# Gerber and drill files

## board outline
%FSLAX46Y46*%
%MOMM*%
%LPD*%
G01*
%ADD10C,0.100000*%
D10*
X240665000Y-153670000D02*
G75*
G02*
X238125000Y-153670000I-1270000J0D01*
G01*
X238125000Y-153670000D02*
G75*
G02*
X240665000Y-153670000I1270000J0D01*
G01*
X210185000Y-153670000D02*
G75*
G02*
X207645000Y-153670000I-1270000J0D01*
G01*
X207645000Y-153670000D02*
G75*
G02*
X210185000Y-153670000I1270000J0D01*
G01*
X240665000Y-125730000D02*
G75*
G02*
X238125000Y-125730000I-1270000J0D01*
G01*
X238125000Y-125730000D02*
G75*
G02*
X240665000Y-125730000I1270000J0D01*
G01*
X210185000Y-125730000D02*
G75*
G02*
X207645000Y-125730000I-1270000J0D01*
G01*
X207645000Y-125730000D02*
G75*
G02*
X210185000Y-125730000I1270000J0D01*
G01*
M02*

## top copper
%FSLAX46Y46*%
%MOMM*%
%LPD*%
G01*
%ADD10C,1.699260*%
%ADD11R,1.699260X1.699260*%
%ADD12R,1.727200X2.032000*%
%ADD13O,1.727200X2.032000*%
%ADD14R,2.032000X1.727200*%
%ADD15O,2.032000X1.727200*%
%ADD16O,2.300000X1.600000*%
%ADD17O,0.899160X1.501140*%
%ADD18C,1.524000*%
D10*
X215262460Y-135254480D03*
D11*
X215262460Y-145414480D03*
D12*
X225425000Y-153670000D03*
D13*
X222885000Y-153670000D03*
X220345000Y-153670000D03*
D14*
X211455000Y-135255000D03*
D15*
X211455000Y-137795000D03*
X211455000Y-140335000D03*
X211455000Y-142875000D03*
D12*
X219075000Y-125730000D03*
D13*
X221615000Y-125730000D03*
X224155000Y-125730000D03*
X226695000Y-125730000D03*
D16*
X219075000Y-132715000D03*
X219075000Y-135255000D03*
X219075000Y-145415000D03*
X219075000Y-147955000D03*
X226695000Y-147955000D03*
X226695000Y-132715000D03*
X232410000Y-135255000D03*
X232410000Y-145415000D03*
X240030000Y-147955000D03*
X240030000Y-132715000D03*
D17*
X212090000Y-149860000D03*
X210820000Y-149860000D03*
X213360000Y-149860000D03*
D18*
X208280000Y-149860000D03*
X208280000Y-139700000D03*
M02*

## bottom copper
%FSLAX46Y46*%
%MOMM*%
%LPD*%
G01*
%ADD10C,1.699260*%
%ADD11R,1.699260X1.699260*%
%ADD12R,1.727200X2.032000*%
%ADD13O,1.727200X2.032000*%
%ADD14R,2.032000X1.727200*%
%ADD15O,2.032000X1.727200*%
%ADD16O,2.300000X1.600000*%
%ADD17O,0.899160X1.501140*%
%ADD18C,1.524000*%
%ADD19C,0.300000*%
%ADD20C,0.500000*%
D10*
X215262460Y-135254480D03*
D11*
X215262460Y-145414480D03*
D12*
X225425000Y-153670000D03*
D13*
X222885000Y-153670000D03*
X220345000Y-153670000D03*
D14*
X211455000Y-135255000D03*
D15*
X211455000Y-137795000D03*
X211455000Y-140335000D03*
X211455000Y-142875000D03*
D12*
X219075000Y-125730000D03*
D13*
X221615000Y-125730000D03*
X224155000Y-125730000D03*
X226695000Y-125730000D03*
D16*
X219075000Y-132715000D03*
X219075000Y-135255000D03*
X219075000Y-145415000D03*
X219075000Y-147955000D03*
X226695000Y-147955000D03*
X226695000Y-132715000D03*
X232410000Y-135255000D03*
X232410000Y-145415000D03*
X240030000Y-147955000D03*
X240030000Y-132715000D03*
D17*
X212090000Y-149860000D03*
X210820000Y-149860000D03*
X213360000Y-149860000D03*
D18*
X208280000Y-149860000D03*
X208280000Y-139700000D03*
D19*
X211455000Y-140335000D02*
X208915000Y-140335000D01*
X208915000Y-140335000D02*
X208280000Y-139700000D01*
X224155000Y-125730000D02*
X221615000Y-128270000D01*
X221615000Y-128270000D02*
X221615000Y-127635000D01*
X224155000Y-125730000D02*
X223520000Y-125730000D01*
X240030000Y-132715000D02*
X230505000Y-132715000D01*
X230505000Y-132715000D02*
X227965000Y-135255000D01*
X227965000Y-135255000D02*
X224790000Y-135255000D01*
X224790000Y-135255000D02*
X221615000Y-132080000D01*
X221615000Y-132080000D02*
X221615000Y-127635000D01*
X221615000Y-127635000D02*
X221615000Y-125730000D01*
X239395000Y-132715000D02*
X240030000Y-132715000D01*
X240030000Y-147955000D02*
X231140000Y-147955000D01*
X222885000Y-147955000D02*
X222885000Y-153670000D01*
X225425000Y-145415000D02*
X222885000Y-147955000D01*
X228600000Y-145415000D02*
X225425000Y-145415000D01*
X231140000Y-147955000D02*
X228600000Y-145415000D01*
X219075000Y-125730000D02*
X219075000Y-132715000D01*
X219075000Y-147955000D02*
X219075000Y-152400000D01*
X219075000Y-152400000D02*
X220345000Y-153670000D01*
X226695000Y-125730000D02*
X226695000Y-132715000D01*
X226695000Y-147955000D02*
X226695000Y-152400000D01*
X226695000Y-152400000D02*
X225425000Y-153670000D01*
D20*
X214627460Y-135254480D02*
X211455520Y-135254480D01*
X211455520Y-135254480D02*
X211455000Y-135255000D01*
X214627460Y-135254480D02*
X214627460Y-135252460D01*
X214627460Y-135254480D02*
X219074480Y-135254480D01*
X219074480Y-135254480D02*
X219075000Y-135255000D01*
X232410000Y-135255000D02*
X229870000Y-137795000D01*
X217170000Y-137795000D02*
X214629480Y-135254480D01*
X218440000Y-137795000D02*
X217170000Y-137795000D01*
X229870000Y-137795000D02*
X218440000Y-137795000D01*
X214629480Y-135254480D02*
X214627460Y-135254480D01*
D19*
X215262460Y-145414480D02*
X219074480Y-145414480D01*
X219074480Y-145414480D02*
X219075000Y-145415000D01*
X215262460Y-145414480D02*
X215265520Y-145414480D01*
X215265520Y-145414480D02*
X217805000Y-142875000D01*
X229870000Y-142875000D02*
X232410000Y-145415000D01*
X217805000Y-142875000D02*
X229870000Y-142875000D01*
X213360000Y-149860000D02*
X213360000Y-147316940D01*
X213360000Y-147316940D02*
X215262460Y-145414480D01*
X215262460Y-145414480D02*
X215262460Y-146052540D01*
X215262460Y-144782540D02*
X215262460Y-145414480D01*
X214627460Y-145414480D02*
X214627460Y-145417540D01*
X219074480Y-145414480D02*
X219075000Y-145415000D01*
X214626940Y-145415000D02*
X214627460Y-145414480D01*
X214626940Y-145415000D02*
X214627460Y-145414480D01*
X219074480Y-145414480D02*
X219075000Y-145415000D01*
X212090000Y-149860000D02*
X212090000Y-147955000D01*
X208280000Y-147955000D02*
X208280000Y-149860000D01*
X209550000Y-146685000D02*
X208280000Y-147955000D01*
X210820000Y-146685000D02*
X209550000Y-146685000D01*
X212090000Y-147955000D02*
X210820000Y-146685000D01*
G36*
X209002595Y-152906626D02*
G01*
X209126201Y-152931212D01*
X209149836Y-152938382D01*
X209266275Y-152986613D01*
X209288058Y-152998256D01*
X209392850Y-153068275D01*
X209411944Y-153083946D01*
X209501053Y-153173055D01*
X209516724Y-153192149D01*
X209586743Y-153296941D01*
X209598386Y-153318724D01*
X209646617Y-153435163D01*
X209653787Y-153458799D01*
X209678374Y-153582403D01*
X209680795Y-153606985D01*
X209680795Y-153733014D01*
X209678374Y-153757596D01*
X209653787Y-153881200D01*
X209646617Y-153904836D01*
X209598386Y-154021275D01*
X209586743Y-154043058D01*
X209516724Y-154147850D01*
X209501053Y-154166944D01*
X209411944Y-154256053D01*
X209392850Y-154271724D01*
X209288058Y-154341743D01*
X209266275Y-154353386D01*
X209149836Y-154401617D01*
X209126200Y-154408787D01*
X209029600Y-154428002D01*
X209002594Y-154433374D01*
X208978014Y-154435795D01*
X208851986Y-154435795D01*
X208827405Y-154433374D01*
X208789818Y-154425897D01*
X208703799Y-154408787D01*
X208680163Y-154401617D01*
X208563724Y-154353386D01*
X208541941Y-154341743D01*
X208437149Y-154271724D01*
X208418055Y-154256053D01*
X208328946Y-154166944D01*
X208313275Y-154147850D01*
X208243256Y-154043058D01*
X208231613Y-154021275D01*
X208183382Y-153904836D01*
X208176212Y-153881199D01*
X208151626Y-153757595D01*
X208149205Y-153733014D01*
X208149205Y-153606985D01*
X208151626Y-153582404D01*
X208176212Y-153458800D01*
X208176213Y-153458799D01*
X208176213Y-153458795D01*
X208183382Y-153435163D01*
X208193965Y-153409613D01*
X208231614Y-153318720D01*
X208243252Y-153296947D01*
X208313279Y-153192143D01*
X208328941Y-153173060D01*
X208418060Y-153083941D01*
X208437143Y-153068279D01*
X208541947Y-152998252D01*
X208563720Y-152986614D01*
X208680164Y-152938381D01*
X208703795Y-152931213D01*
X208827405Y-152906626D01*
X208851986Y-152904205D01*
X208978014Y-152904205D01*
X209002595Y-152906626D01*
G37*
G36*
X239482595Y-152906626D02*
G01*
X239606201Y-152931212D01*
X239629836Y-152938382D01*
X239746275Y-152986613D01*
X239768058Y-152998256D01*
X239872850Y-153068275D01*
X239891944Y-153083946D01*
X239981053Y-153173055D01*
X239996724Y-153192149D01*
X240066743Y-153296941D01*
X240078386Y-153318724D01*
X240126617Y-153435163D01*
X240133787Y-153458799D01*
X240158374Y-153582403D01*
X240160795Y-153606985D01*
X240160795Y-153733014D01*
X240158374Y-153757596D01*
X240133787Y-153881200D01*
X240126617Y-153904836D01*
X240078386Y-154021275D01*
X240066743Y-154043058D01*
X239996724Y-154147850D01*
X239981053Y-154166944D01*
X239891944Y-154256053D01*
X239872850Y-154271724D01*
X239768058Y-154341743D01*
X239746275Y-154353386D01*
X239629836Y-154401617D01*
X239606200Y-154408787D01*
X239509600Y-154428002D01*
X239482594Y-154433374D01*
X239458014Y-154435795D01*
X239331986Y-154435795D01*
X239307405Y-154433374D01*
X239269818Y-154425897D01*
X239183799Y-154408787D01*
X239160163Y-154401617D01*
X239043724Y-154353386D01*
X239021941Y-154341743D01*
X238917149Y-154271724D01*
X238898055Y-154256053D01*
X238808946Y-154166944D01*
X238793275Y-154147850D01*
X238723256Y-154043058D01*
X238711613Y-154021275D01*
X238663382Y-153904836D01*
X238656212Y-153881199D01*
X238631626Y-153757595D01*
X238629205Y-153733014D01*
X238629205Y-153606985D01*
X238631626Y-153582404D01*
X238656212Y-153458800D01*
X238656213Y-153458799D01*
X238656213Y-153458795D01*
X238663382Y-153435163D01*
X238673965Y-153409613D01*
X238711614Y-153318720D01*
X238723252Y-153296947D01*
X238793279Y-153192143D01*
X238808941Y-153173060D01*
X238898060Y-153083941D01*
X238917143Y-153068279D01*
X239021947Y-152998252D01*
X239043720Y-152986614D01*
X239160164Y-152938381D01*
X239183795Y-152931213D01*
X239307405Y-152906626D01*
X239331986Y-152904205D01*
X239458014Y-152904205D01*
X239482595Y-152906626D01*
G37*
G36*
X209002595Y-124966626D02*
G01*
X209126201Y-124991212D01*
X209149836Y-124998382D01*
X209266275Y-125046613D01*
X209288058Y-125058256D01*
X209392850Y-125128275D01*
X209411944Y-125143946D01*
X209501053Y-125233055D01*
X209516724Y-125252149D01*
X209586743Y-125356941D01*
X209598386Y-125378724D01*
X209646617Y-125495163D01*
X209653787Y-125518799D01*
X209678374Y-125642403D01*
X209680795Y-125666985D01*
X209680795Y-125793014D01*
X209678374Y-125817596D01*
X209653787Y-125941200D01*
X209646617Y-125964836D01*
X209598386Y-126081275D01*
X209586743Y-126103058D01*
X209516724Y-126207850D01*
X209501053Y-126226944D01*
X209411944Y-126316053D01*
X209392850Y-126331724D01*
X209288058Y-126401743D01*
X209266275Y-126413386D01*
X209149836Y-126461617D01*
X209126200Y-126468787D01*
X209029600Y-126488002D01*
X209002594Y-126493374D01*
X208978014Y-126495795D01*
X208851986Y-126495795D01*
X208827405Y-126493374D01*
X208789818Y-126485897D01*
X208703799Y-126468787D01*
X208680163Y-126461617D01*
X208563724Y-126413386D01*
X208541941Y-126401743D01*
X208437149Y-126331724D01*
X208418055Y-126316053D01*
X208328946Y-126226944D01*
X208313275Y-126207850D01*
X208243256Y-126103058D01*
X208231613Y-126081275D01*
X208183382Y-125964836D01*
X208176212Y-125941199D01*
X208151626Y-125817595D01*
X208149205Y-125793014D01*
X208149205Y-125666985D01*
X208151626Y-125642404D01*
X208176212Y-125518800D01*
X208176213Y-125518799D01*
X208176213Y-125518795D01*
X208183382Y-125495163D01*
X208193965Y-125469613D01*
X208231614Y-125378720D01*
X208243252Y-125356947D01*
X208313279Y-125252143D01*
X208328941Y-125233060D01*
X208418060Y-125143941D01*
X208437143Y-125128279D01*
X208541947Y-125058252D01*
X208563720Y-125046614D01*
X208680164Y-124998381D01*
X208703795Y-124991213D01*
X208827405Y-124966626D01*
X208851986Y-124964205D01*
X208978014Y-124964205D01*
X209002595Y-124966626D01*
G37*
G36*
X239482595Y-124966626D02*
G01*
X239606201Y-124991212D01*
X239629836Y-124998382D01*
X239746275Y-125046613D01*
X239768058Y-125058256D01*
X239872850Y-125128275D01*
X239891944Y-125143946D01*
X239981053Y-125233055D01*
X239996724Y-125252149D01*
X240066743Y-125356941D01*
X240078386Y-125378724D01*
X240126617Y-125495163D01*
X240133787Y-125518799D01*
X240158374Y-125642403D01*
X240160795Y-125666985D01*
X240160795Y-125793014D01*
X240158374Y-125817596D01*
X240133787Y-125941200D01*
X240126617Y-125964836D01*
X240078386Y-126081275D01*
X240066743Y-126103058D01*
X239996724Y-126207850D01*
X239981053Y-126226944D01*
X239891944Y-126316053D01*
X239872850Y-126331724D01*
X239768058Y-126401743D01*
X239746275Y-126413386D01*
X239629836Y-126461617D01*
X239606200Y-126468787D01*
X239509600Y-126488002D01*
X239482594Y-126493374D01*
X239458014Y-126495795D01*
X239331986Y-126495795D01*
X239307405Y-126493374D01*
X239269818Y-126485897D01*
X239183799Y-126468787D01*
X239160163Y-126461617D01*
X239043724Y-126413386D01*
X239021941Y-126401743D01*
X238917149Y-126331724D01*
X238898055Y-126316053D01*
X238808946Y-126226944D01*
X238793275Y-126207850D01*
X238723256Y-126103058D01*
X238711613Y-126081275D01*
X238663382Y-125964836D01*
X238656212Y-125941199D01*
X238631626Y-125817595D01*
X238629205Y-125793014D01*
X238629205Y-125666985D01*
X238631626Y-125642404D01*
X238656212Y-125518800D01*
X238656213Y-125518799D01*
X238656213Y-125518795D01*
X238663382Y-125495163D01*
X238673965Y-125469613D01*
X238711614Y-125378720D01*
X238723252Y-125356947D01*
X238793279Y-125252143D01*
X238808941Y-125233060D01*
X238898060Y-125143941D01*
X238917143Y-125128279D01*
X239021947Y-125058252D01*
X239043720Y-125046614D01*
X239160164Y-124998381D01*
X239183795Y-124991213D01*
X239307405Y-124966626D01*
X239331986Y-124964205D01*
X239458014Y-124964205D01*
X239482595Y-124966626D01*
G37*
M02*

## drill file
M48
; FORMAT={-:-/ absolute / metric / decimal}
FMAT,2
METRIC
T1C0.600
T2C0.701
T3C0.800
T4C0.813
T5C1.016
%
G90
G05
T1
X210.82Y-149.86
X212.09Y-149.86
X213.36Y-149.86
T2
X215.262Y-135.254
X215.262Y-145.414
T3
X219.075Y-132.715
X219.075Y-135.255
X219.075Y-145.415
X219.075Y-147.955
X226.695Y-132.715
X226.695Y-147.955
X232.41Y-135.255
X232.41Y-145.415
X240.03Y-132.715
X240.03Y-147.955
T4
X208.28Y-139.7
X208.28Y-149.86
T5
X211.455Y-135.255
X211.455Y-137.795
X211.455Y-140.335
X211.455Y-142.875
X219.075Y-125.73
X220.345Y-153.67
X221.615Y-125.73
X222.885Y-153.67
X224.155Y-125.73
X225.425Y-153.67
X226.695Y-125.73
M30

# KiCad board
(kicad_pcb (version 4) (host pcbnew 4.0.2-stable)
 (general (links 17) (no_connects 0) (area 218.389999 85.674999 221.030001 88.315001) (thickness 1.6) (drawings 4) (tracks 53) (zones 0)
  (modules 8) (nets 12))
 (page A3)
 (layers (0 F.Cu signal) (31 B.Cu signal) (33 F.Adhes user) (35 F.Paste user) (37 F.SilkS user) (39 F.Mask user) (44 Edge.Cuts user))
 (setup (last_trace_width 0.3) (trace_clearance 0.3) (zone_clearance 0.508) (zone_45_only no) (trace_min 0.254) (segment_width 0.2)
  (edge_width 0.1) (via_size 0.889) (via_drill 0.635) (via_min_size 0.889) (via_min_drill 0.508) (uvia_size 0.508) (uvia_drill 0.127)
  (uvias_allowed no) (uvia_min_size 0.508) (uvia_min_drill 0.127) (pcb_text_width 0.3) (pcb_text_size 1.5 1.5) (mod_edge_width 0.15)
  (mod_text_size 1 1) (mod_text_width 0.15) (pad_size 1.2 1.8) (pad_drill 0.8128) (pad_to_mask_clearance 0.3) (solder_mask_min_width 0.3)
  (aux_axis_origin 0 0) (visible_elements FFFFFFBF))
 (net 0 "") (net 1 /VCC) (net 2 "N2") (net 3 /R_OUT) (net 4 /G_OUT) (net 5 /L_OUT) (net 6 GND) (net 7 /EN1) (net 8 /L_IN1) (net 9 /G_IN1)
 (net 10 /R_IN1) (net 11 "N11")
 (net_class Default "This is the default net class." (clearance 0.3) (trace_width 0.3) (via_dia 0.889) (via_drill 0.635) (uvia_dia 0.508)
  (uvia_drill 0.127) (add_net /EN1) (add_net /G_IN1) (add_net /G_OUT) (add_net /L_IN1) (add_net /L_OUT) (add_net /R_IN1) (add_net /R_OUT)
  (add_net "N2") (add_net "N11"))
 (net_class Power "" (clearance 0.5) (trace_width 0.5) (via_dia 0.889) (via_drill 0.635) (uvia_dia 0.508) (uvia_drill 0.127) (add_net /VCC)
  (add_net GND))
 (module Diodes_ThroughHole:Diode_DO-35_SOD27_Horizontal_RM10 (layer F.Cu) (at 215.265 145.415 90)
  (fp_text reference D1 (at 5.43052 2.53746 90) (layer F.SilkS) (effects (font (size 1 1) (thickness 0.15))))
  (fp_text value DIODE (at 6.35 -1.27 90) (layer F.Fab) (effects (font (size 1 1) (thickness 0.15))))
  (pad 2 thru_hole circle (at 10.16052 -0.00254 270) (size 1.69926 1.69926) (drill 0.70104) (layers *.Cu *.Mask F.SilkS) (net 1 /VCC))
  (pad 1 thru_hole rect (at 0.00052 -0.00254 270) (size 1.69926 1.69926) (drill 0.70104) (layers *.Cu *.Mask F.SilkS) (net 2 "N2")))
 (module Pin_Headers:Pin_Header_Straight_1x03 (layer F.Cu) (at 225.425 153.67 270)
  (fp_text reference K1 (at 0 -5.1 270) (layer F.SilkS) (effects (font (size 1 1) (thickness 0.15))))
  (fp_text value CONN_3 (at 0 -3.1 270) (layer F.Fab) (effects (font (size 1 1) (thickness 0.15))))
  (pad 1 thru_hole rect (at 0 0 270) (size 2.032 1.7272) (drill 1.016) (layers *.Cu *.Mask F.SilkS) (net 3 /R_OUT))
  (pad 2 thru_hole oval (at 0 2.54 270) (size 2.032 1.7272) (drill 1.016) (layers *.Cu *.Mask F.SilkS) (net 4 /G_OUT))
  (pad 3 thru_hole oval (at 0 5.08 270) (size 2.032 1.7272) (drill 1.016) (layers *.Cu *.Mask F.SilkS) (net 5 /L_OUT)))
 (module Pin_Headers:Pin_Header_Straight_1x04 (layer F.Cu) (at 211.455 135.255)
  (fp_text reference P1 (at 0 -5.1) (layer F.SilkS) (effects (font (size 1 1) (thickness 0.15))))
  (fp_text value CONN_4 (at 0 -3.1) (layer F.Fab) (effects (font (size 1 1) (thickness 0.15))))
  (pad 1 thru_hole rect (at 0 0) (size 2.032 1.7272) (drill 1.016) (layers *.Cu *.Mask F.SilkS) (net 1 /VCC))
  (pad 2 thru_hole oval (at 0 2.54) (size 2.032 1.7272) (drill 1.016) (layers *.Cu *.Mask F.SilkS) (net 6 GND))
  (pad 3 thru_hole oval (at 0 5.08) (size 2.032 1.7272) (drill 1.016) (layers *.Cu *.Mask F.SilkS) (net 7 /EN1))
  (pad 4 thru_hole oval (at 0 7.62) (size 2.032 1.7272) (drill 1.016) (layers *.Cu *.Mask F.SilkS) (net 6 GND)))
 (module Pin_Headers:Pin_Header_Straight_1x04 (layer F.Cu) (at 219.075 125.73 90)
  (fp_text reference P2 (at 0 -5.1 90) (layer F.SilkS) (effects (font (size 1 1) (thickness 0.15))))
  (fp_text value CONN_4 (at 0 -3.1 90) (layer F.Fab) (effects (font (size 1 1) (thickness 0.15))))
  (pad 1 thru_hole rect (at 0 0 90) (size 2.032 1.7272) (drill 1.016) (layers *.Cu *.Mask F.SilkS) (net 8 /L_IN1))
  (pad 2 thru_hole oval (at 0 2.54 90) (size 2.032 1.7272) (drill 1.016) (layers *.Cu *.Mask F.SilkS) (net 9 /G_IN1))
  (pad 3 thru_hole oval (at 0 5.08 90) (size 2.032 1.7272) (drill 1.016) (layers *.Cu *.Mask F.SilkS) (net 9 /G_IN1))
  (pad 4 thru_hole oval (at 0 7.62 90) (size 2.032 1.7272) (drill 1.016) (layers *.Cu *.Mask F.SilkS) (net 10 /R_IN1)))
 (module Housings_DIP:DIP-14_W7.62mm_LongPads (layer F.Cu) (at 219.075 132.715)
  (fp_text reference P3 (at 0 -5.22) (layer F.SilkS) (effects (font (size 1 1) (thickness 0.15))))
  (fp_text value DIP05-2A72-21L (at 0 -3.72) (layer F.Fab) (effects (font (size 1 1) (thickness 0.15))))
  (pad 1 thru_hole oval (at 0 0) (size 2.3 1.6) (drill 0.8) (layers *.Cu *.Mask F.SilkS) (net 8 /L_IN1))
  (pad 2 thru_hole oval (at 0 2.54) (size 2.3 1.6) (drill 0.8) (layers *.Cu *.Mask F.SilkS) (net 1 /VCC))
  (pad 6 thru_hole oval (at 0 12.7) (size 2.3 1.6) (drill 0.8) (layers *.Cu *.Mask F.SilkS) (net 2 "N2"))
  (pad 7 thru_hole oval (at 0 15.24) (size 2.3 1.6) (drill 0.8) (layers *.Cu *.Mask F.SilkS) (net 5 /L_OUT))
  (pad 8 thru_hole oval (at 7.62 15.24) (size 2.3 1.6) (drill 0.8) (layers *.Cu *.Mask F.SilkS) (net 3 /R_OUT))
  (pad 14 thru_hole oval (at 7.62 0) (size 2.3 1.6) (drill 0.8) (layers *.Cu *.Mask F.SilkS) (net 10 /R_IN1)))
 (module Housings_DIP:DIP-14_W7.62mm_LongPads (layer F.Cu) (at 232.41 132.715)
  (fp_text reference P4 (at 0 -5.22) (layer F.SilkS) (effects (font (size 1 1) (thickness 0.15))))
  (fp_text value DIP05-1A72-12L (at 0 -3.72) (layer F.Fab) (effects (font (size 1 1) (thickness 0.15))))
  (pad 2 thru_hole oval (at 0 2.54) (size 2.3 1.6) (drill 0.8) (layers *.Cu *.Mask F.SilkS) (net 1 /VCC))
  (pad 6 thru_hole oval (at 0 12.7) (size 2.3 1.6) (drill 0.8) (layers *.Cu *.Mask F.SilkS) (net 2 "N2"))
  (pad 8 thru_hole oval (at 7.62 15.24) (size 2.3 1.6) (drill 0.8) (layers *.Cu *.Mask F.SilkS) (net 4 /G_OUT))
  (pad 14 thru_hole oval (at 7.62 0) (size 2.3 1.6) (drill 0.8) (layers *.Cu *.Mask F.SilkS) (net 9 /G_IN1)))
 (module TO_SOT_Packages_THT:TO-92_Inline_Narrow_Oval (layer F.Cu) (at 213.36 149.86 180)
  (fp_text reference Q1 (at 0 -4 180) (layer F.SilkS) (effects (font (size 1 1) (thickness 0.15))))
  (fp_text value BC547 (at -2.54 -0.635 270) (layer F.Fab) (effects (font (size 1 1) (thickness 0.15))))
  (pad 2 thru_hole oval (at 1.27 0) (size 0.89916 1.50114) (drill 0.6) (layers *.Cu *.Mask F.SilkS) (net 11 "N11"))
  (pad 3 thru_hole oval (at 2.54 0) (size 0.89916 1.50114) (drill 0.6) (layers *.Cu *.Mask F.SilkS) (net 6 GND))
  (pad 1 thru_hole oval (at 0 0) (size 0.89916 1.50114) (drill 0.6) (layers *.Cu *.Mask F.SilkS) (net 2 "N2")))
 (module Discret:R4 (layer F.Cu) (at 208.28 144.78 90)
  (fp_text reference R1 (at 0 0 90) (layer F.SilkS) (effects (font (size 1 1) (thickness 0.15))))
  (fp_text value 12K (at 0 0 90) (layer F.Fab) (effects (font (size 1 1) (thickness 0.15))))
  (pad 1 thru_hole circle (at -5.08 0 90) (size 1.524 1.524) (drill 0.8128) (layers *.Cu *.Mask F.SilkS) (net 11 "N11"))
  (pad 2 thru_hole circle (at 5.08 0 90) (size 1.524 1.524) (drill 0.8128) (layers *.Cu *.Mask F.SilkS) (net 7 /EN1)))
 (gr_circle (center 239.395 153.67) (end 240.665 153.67) (layer Edge.Cuts) (width 0.1))
 (gr_circle (center 208.915 153.67) (end 210.185 153.67) (layer Edge.Cuts) (width 0.1))
 (gr_circle (center 239.395 125.73) (end 240.665 125.73) (layer Edge.Cuts) (width 0.1))
 (gr_circle (center 208.915 125.73) (end 210.185 125.73) (layer Edge.Cuts) (width 0.1))
 (segment (start 211.455 140.335) (end 208.915 140.335) (width 0.3) (layer B.Cu) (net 7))
 (segment (start 208.915 140.335) (end 208.28 139.7) (width 0.3) (layer B.Cu) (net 7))
 (segment (start 224.155 125.73) (end 221.615 128.27) (width 0.3) (layer B.Cu) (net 9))
 (segment (start 221.615 128.27) (end 221.615 127.635) (width 0.3) (layer B.Cu) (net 9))
 (segment (start 224.155 125.73) (end 223.52 125.73) (width 0.3) (layer B.Cu) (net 9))
 (segment (start 240.03 132.715) (end 230.505 132.715) (width 0.3) (layer B.Cu) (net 9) (status 400000))
 (segment (start 230.505 132.715) (end 227.965 135.255) (width 0.3) (layer B.Cu) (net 9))
 (segment (start 227.965 135.255) (end 224.79 135.255) (width 0.3) (layer B.Cu) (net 9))
 (segment (start 224.79 135.255) (end 221.615 132.08) (width 0.3) (layer B.Cu) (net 9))
 (segment (start 221.615 132.08) (end 221.615 127.635) (width 0.3) (layer B.Cu) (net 9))
 (segment (start 221.615 127.635) (end 221.615 125.73) (width 0.3) (layer B.Cu) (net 9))
 (segment (start 239.395 132.715) (end 240.03 132.715) (width 0.3) (layer B.Cu) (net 9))
 (segment (start 240.03 147.955) (end 231.14 147.955) (width 0.3) (layer B.Cu) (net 4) (status 400000))
 (segment (start 222.885 147.955) (end 222.885 153.67) (width 0.3) (layer B.Cu) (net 4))
 (segment (start 225.425 145.415) (end 222.885 147.955) (width 0.3) (layer B.Cu) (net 4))
 (segment (start 228.6 145.415) (end 225.425 145.415) (width 0.3) (layer B.Cu) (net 4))
 (segment (start 231.14 147.955) (end 228.6 145.415) (width 0.3) (layer B.Cu) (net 4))
 (segment (start 219.075 125.73) (end 219.075 132.715) (width 0.3) (layer B.Cu) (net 8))
 (segment (start 219.075 147.955) (end 219.075 152.4) (width 0.3) (layer B.Cu) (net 5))
 (segment (start 219.075 152.4) (end 220.345 153.67) (width 0.3) (layer B.Cu) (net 5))
 (segment (start 226.695 125.73) (end 226.695 132.715) (width 0.3) (layer B.Cu) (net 10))
 (segment (start 226.695 147.955) (end 226.695 152.4) (width 0.3) (layer B.Cu) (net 3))
 (segment (start 226.695 152.4) (end 225.425 153.67) (width 0.3) (layer B.Cu) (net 3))
 (segment (start 214.62746 135.25448) (end 211.45552 135.25448) (width 0.5) (layer B.Cu) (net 1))
 (segment (start 211.45552 135.25448) (end 211.455 135.255) (width 0.5) (layer B.Cu) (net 1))
 (segment (start 214.62746 135.25448) (end 214.62746 135.25246) (width 0.5) (layer B.Cu) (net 1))
 (segment (start 214.62746 135.25448) (end 219.07448 135.25448) (width 0.5) (layer B.Cu) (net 1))
 (segment (start 219.07448 135.25448) (end 219.075 135.255) (width 0.5) (layer B.Cu) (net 1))
 (segment (start 232.41 135.255) (end 229.87 137.795) (width 0.5) (layer B.Cu) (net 1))
 (segment (start 217.17 137.795) (end 214.62948 135.25448) (width 0.5) (layer B.Cu) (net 1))
 (segment (start 218.44 137.795) (end 217.17 137.795) (width 0.5) (layer B.Cu) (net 1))
 (segment (start 229.87 137.795) (end 218.44 137.795) (width 0.5) (layer B.Cu) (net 1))
 (segment (start 214.62948 135.25448) (end 214.62746 135.25448) (width 0.5) (layer B.Cu) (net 1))
 (segment (start 215.26246 145.41448) (end 219.07448 145.41448) (width 0.3) (layer B.Cu) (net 2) (status C00000))
 (segment (start 219.07448 145.41448) (end 219.075 145.415) (width 0.3) (layer B.Cu) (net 2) (status C00000))
 (segment (start 215.26246 145.41448) (end 215.26552 145.41448) (width 0.3) (layer B.Cu) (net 2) (status C00000))
 (segment (start 215.26552 145.41448) (end 217.805 142.875) (width 0.3) (layer B.Cu) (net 2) (status 400000))
 (segment (start 229.87 142.875) (end 232.41 145.415) (width 0.3) (layer B.Cu) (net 2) (status 800000))
 (segment (start 217.805 142.875) (end 229.87 142.875) (width 0.3) (layer B.Cu) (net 2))
 (segment (start 213.36 149.86) (end 213.36 147.31694) (width 0.3) (layer B.Cu) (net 2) (status 400000))
 (segment (start 213.36 147.31694) (end 215.26246 145.41448) (width 0.3) (layer B.Cu) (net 2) (status 800000))
 (segment (start 215.26246 145.41448) (end 215.26246 146.05254) (width 0.3) (layer B.Cu) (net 2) (status C00000))
 (segment (start 215.26246 144.78254) (end 215.26246 145.41448) (width 0.3) (layer B.Cu) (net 2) (status C00000))
 (segment (start 214.62746 145.41448) (end 214.62746 145.41754) (width 0.3) (layer B.Cu) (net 2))
 (segment (start 219.07448 145.41448) (end 219.075 145.415) (width 0.3) (layer B.Cu) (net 2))
 (segment (start 214.62694 145.415) (end 214.62746 145.41448) (width 0.3) (layer B.Cu) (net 2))
 (segment (start 214.62694 145.415) (end 214.62746 145.41448) (width 0.3) (layer B.Cu) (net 2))
 (segment (start 219.07448 145.41448) (end 219.075 145.415) (width 0.3) (layer B.Cu) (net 2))
 (segment (start 212.09 149.86) (end 212.09 147.955) (width 0.3) (layer B.Cu) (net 11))
 (segment (start 208.28 147.955) (end 208.28 149.86) (width 0.3) (layer B.Cu) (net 11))
 (segment (start 209.55 146.685) (end 208.28 147.955) (width 0.3) (layer B.Cu) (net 11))
 (segment (start 210.82 146.685) (end 209.55 146.685) (width 0.3) (layer B.Cu) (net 11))
 (segment (start 212.09 147.955) (end 210.82 146.685) (width 0.3) (layer B.Cu) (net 11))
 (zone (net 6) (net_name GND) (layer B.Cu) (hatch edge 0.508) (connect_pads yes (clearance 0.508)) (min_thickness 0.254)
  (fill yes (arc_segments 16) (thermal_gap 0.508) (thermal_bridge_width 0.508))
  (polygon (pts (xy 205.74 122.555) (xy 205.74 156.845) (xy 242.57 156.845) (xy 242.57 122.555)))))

